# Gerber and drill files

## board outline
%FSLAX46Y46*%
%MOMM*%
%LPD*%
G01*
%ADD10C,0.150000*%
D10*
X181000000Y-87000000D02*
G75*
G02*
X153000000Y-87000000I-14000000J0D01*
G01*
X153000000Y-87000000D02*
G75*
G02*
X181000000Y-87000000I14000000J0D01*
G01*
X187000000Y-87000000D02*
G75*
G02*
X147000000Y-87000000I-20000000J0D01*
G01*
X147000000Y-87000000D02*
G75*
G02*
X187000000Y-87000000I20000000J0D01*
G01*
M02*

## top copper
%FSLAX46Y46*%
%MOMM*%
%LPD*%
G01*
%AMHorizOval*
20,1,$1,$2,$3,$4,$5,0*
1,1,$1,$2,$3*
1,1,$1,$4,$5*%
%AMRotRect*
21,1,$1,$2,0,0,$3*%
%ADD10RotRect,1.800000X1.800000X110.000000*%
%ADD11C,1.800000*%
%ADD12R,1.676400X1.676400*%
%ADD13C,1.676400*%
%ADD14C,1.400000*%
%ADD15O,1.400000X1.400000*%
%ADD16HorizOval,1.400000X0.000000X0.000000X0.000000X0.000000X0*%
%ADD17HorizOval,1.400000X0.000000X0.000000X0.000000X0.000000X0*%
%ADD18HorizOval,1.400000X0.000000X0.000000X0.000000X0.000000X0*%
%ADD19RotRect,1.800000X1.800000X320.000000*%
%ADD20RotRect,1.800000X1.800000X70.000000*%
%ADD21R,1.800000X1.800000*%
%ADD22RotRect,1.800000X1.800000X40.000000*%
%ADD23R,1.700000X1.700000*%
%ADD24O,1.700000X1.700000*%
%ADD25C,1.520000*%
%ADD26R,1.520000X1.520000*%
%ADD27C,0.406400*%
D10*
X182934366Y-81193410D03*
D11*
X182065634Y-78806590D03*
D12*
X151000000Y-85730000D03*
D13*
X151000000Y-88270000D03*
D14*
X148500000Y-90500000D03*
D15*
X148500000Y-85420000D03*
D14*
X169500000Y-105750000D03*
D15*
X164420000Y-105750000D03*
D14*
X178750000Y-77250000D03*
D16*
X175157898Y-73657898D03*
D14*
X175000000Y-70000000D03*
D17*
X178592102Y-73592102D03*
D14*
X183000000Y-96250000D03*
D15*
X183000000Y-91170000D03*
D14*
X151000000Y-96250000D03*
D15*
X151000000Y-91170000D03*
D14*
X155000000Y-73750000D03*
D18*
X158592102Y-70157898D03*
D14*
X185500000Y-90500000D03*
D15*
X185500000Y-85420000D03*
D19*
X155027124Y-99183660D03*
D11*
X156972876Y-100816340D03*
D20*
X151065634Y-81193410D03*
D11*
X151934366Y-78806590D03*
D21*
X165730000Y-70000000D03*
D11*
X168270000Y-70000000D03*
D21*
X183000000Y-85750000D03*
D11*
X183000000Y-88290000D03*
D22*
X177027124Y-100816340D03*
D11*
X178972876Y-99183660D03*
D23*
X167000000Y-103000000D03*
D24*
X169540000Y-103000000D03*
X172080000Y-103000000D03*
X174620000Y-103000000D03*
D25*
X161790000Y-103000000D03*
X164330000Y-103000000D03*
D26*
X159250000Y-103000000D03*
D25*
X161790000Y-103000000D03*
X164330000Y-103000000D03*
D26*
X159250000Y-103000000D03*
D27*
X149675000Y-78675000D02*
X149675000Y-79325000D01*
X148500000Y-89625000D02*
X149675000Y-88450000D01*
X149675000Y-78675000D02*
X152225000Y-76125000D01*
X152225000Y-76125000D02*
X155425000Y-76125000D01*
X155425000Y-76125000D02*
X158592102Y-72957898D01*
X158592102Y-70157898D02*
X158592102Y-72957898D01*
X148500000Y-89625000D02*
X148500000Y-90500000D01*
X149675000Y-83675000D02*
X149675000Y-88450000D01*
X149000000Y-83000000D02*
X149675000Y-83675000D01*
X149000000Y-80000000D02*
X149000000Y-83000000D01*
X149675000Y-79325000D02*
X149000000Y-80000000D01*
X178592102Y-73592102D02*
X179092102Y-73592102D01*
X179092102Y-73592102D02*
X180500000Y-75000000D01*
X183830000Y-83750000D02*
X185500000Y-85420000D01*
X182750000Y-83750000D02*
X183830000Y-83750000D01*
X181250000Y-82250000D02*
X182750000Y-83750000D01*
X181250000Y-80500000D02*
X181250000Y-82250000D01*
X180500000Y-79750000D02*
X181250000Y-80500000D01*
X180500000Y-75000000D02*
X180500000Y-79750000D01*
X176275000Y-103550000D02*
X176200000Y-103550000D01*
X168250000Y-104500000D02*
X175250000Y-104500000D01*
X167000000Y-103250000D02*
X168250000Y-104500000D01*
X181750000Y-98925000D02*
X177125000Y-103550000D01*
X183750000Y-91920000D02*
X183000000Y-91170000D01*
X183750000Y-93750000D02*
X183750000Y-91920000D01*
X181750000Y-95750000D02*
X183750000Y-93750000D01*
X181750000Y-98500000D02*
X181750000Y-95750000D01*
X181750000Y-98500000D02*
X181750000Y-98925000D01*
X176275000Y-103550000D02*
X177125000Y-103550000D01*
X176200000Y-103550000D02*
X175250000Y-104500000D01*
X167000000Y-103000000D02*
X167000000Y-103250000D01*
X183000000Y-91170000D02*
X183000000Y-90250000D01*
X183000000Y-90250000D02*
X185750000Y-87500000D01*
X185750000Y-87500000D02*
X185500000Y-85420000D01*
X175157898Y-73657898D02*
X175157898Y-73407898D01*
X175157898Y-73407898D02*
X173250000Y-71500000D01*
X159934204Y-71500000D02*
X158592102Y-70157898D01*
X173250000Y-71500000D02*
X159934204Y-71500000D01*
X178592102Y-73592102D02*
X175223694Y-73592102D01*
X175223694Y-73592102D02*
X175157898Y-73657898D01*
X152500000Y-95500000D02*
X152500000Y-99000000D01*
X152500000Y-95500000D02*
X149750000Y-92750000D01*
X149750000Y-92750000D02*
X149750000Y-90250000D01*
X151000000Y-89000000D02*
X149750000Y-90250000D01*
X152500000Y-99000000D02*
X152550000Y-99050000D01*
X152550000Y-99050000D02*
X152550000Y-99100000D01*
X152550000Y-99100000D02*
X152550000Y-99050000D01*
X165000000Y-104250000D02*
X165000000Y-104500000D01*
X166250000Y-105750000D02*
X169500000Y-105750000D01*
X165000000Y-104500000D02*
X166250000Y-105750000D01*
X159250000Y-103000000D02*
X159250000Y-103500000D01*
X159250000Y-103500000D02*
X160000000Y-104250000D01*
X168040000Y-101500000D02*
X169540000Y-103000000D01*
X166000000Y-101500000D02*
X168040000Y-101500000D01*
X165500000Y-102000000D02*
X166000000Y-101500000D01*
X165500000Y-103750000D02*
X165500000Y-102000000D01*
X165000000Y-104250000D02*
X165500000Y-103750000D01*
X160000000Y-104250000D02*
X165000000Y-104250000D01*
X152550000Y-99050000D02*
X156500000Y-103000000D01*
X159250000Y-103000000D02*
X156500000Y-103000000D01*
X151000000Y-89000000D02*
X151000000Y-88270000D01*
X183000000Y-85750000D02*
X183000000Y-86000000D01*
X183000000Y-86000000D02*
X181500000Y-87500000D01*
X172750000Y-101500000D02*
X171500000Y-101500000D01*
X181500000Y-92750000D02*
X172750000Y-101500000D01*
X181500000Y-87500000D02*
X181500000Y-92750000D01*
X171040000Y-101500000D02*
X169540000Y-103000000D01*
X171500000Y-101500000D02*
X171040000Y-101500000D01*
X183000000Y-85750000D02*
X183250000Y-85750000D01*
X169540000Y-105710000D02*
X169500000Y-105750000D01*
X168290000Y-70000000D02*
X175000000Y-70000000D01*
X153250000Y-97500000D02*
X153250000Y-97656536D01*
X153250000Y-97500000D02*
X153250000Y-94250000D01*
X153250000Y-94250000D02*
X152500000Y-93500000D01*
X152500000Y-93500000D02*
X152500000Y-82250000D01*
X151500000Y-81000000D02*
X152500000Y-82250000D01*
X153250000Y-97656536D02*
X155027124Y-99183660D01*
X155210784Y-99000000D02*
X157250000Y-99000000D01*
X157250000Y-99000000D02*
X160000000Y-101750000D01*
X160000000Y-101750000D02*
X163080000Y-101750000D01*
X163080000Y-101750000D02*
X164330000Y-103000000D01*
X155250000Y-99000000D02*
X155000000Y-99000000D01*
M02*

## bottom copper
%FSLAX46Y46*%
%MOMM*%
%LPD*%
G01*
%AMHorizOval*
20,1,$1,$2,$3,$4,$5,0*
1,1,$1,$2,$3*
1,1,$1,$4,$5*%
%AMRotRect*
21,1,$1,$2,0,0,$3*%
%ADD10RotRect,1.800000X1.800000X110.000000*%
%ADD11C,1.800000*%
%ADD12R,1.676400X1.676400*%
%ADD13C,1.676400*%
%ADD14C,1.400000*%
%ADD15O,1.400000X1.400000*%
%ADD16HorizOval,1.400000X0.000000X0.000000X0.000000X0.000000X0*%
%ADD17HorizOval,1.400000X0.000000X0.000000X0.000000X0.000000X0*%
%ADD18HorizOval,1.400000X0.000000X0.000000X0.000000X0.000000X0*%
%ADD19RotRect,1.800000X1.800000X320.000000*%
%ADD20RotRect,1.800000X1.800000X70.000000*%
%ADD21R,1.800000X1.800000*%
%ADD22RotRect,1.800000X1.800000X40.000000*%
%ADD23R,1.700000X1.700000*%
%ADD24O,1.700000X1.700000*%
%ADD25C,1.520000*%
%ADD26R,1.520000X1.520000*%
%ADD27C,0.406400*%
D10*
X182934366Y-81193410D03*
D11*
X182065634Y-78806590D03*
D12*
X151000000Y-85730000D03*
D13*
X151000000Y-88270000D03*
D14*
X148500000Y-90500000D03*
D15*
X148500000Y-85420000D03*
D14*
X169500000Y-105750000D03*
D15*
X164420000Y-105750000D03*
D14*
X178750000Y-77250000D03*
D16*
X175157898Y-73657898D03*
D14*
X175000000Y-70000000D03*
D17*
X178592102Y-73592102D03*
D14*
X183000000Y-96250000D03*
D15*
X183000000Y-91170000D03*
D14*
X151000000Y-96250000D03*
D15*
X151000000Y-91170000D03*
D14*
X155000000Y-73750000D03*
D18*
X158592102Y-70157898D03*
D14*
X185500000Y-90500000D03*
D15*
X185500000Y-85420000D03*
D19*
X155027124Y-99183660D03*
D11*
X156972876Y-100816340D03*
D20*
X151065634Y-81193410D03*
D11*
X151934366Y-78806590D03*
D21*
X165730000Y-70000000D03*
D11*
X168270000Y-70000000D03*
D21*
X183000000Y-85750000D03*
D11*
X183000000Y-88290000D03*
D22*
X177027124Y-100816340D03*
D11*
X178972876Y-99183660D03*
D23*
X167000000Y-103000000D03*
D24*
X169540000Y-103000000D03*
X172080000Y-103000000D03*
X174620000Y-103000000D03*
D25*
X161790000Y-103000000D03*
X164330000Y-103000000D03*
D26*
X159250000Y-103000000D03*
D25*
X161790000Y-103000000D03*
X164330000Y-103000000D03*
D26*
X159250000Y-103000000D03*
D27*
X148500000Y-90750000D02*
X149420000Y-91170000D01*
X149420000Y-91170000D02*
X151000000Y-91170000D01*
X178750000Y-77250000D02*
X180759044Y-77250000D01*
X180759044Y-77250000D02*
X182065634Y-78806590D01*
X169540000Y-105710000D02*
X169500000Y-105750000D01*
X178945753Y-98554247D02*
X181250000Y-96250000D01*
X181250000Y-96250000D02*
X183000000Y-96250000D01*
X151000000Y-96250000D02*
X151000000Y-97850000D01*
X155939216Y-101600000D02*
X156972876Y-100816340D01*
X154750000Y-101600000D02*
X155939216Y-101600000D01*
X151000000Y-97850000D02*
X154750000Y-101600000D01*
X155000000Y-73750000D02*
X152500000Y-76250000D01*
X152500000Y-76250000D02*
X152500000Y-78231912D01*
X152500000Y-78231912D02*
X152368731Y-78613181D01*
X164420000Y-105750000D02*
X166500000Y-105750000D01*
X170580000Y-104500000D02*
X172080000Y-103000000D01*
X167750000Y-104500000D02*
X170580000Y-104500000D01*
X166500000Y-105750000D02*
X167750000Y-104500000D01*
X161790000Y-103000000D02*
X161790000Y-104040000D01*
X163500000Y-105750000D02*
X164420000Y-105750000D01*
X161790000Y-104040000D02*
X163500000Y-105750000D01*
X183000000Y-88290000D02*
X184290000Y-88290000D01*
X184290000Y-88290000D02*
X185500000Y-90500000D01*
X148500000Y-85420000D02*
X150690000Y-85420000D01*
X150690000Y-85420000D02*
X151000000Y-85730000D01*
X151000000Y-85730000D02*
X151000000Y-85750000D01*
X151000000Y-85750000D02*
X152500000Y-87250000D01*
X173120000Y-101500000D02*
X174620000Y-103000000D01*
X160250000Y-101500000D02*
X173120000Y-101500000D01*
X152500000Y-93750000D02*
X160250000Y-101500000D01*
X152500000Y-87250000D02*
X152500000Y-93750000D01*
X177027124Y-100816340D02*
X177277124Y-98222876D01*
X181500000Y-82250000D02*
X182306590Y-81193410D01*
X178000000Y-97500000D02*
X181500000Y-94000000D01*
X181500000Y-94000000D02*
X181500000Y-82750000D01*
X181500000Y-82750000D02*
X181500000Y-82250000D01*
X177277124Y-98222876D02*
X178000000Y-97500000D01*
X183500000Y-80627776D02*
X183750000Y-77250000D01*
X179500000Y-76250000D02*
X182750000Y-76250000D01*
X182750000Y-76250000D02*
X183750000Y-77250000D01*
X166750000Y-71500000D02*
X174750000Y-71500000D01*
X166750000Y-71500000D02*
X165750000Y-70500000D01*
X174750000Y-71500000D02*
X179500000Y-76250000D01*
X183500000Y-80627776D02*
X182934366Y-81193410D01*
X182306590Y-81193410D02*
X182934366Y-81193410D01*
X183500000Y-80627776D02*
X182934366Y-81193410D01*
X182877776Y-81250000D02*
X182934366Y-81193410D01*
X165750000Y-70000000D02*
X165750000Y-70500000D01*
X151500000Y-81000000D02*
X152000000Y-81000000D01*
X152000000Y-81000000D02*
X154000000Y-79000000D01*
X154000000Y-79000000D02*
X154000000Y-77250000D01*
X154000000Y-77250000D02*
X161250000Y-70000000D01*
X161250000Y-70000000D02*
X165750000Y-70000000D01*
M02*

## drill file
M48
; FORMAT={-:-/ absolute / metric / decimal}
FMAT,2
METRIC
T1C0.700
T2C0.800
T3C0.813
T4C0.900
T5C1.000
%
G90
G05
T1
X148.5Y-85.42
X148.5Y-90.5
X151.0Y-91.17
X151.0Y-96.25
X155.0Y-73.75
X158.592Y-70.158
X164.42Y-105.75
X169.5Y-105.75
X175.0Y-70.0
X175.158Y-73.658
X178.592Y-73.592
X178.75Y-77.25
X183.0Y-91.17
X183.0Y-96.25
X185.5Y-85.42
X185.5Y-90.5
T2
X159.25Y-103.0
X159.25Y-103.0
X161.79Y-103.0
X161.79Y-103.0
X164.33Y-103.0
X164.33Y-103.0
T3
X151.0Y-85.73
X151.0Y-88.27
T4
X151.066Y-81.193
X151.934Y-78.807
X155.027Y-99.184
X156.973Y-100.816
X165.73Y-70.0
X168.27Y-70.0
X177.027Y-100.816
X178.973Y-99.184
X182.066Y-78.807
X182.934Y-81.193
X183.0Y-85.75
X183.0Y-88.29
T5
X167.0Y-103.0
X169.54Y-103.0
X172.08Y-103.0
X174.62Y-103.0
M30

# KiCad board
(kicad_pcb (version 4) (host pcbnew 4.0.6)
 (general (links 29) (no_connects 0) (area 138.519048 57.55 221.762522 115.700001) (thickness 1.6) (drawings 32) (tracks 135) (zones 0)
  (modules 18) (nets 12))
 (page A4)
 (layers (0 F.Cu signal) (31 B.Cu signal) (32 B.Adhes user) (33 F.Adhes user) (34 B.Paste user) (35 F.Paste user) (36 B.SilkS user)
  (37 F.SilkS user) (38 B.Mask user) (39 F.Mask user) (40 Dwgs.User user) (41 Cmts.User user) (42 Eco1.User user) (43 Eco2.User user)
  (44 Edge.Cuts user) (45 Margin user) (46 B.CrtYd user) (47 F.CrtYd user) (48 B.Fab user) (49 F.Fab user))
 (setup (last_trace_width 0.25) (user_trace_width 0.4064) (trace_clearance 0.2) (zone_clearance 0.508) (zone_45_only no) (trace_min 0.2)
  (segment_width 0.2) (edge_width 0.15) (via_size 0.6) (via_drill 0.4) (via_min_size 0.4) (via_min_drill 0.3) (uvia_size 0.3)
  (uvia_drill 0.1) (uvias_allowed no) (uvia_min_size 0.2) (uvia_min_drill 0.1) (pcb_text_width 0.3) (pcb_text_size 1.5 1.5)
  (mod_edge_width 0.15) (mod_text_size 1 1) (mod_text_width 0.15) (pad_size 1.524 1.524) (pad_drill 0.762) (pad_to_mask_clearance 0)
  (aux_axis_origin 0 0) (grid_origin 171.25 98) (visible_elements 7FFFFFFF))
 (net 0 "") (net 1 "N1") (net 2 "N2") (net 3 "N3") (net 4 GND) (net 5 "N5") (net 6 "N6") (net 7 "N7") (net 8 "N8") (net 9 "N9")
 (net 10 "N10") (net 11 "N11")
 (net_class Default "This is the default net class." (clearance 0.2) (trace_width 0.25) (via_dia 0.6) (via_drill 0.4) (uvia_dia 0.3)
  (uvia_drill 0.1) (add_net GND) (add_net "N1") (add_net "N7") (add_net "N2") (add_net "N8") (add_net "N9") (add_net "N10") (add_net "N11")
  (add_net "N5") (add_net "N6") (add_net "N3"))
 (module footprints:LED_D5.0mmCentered (layer F.Cu) (at 182.5 80 110)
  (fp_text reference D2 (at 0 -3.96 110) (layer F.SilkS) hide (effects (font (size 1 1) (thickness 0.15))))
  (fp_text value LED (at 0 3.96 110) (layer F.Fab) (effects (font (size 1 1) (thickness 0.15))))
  (pad 1 thru_hole rect (at -1.27 0 110) (size 1.8 1.8) (drill 0.9) (layers *.Cu *.Mask) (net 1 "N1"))
  (pad 2 thru_hole circle (at 1.27 0 110) (size 1.8 1.8) (drill 0.9) (layers *.Cu *.Mask) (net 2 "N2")))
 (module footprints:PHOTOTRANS (layer F.Cu) (at 151 87 270)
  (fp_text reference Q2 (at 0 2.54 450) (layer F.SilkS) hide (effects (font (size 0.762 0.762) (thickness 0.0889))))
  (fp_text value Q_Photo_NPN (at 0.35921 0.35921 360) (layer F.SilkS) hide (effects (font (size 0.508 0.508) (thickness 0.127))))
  (pad 1 thru_hole rect (at -1.27 0 270) (size 1.6764 1.6764) (drill 0.8128) (layers *.Cu *.Mask F.SilkS) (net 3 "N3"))
  (pad 2 thru_hole circle (at 1.27 0 315) (size 1.6764 1.6764) (drill 0.8128) (layers *.Cu *.Mask F.SilkS) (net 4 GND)))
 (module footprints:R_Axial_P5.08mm (layer F.Cu) (at 148.5 90.5 90)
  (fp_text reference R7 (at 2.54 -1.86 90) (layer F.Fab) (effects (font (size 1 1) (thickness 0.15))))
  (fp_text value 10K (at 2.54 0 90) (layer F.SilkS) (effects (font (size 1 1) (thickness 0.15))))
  (pad 1 thru_hole circle (at 0 0 90) (size 1.4 1.4) (drill 0.7) (layers *.Cu *.Mask) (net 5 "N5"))
  (pad 2 thru_hole oval (at 5.08 0 90) (size 1.4 1.4) (drill 0.7) (layers *.Cu *.Mask) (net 3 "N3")))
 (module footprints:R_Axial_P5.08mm (layer F.Cu) (at 169.5 105.75 180)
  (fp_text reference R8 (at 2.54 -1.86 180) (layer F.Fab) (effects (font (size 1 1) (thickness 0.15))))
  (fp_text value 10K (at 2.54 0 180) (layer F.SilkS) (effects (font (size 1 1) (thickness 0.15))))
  (pad 1 thru_hole circle (at 0 0 180) (size 1.4 1.4) (drill 0.7) (layers *.Cu *.Mask) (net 4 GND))
  (pad 2 thru_hole oval (at 5.08 0 180) (size 1.4 1.4) (drill 0.7) (layers *.Cu *.Mask) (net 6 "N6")))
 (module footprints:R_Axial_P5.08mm (layer F.Cu) (at 178.75 77.25 135)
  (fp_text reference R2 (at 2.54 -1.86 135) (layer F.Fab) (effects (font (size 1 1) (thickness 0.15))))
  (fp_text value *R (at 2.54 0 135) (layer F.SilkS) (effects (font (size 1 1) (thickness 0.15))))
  (pad 1 thru_hole circle (at 0 0 135) (size 1.4 1.4) (drill 0.7) (layers *.Cu *.Mask) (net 2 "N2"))
  (pad 2 thru_hole oval (at 5.08 0 135) (size 1.4 1.4) (drill 0.7) (layers *.Cu *.Mask) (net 5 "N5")))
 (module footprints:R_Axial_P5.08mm (layer F.Cu) (at 175 70 315)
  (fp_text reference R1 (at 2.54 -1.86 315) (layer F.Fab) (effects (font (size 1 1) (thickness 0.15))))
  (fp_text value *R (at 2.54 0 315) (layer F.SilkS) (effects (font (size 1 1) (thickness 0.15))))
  (pad 1 thru_hole circle (at 0 0 315) (size 1.4 1.4) (drill 0.7) (layers *.Cu *.Mask) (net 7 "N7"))
  (pad 2 thru_hole oval (at 5.08 0 315) (size 1.4 1.4) (drill 0.7) (layers *.Cu *.Mask) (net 5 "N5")))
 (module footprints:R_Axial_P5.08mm (layer F.Cu) (at 183 96.25 90)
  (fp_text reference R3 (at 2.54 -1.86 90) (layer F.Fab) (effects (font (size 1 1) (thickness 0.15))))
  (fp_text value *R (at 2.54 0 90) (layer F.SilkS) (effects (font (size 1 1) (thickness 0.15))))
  (pad 1 thru_hole circle (at 0 0 90) (size 1.4 1.4) (drill 0.7) (layers *.Cu *.Mask) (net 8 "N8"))
  (pad 2 thru_hole oval (at 5.08 0 90) (size 1.4 1.4) (drill 0.7) (layers *.Cu *.Mask) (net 5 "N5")))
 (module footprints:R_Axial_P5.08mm (layer F.Cu) (at 151 96.25 90)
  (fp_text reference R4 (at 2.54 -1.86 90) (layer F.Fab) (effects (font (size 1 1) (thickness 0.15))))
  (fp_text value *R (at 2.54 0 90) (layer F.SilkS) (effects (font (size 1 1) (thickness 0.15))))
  (pad 1 thru_hole circle (at 0 0 90) (size 1.4 1.4) (drill 0.7) (layers *.Cu *.Mask) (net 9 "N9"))
  (pad 2 thru_hole oval (at 5.08 0 90) (size 1.4 1.4) (drill 0.7) (layers *.Cu *.Mask) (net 5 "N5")))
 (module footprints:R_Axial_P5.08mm (layer F.Cu) (at 155 73.75 45)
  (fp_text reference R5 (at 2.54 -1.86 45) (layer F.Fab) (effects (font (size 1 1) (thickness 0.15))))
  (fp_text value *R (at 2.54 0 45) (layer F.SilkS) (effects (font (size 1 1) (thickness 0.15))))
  (pad 1 thru_hole circle (at 0 0 45) (size 1.4 1.4) (drill 0.7) (layers *.Cu *.Mask) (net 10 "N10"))
  (pad 2 thru_hole oval (at 5.08 0 45) (size 1.4 1.4) (drill 0.7) (layers *.Cu *.Mask) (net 5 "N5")))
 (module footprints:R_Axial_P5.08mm (layer F.Cu) (at 185.5 90.5 90)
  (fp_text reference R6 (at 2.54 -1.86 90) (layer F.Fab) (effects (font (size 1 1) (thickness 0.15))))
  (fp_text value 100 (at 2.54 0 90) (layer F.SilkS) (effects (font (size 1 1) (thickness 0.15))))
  (pad 1 thru_hole circle (at 0 0 90) (size 1.4 1.4) (drill 0.7) (layers *.Cu *.Mask) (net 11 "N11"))
  (pad 2 thru_hole oval (at 5.08 0 90) (size 1.4 1.4) (drill 0.7) (layers *.Cu *.Mask) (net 5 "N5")))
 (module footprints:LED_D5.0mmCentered (layer F.Cu) (at 156 100 320)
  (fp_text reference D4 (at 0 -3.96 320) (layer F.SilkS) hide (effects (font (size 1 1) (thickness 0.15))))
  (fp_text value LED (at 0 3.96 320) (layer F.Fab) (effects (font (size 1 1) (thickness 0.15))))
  (pad 1 thru_hole rect (at -1.27 0 320) (size 1.8 1.8) (drill 0.9) (layers *.Cu *.Mask) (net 1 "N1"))
  (pad 2 thru_hole circle (at 1.27 0 320) (size 1.8 1.8) (drill 0.9) (layers *.Cu *.Mask) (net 9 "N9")))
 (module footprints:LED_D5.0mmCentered (layer F.Cu) (at 151.5 80 70)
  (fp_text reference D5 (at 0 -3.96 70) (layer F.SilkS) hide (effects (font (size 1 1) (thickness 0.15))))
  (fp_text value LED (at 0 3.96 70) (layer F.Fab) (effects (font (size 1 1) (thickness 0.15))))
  (pad 1 thru_hole rect (at -1.27 0 70) (size 1.8 1.8) (drill 0.9) (layers *.Cu *.Mask) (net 1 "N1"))
  (pad 2 thru_hole circle (at 1.27 0 70) (size 1.8 1.8) (drill 0.9) (layers *.Cu *.Mask) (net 10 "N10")))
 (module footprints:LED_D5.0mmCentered (layer F.Cu) (at 167 70)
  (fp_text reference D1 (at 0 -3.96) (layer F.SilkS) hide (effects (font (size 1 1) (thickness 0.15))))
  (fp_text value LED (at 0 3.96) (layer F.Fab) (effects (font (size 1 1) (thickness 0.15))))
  (pad 1 thru_hole rect (at -1.27 0) (size 1.8 1.8) (drill 0.9) (layers *.Cu *.Mask) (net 1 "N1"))
  (pad 2 thru_hole circle (at 1.27 0) (size 1.8 1.8) (drill 0.9) (layers *.Cu *.Mask) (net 7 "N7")))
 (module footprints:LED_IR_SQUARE (layer F.Cu) (at 183 85.75 270)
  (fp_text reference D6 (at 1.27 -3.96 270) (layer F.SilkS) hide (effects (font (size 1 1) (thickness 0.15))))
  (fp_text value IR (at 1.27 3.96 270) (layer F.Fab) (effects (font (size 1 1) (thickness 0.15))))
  (pad 1 thru_hole rect (at 0 0 270) (size 1.8 1.8) (drill 0.9) (layers *.Cu *.Mask) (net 4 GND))
  (pad 2 thru_hole circle (at 2.54 0 270) (size 1.8 1.8) (drill 0.9) (layers *.Cu *.Mask) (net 11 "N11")))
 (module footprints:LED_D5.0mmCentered (layer F.Cu) (at 178 100 40)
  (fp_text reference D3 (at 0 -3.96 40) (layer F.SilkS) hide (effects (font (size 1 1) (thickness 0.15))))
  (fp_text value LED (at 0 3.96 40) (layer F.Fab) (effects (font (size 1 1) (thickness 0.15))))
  (pad 1 thru_hole rect (at -1.27 0 40) (size 1.8 1.8) (drill 0.9) (layers *.Cu *.Mask) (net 1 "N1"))
  (pad 2 thru_hole circle (at 1.27 0 40) (size 1.8 1.8) (drill 0.9) (layers *.Cu *.Mask) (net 8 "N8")))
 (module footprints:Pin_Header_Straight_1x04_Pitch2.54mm (layer F.Cu) (at 167 103 90)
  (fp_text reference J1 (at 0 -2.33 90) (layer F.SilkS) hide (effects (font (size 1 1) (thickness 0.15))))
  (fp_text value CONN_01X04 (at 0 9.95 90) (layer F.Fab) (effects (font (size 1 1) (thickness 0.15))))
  (pad 1 thru_hole rect (at 0 0 90) (size 1.7 1.7) (drill 1) (layers *.Cu *.Mask) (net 5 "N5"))
  (pad 2 thru_hole oval (at 0 2.54 90) (size 1.7 1.7) (drill 1) (layers *.Cu *.Mask) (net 4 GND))
  (pad 3 thru_hole oval (at 0 5.08 90) (size 1.7 1.7) (drill 1) (layers *.Cu *.Mask) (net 6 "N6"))
  (pad 4 thru_hole oval (at 0 7.62 90) (size 1.7 1.7) (drill 1) (layers *.Cu *.Mask) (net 3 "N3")))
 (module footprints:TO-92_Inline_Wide (layer B.Cu) (at 159.25 103)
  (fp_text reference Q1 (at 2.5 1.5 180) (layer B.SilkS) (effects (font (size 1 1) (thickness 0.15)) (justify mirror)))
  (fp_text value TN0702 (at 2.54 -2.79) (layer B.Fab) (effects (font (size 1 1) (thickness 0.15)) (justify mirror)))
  (pad 2 thru_hole circle (at 2.54 0 270) (size 1.52 1.52) (drill 0.8) (layers *.Cu *.Mask) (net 6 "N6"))
  (pad 3 thru_hole circle (at 5.08 0 270) (size 1.52 1.52) (drill 0.8) (layers *.Cu *.Mask) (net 1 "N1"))
  (pad 1 thru_hole rect (at 0 0 270) (size 1.52 1.52) (drill 0.8) (layers *.Cu *.Mask) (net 4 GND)))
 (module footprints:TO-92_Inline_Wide (layer F.Cu) (at 159.25 103)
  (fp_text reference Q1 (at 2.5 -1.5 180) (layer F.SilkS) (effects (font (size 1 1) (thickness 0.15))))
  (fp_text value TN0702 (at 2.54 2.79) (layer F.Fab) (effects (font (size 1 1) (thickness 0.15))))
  (pad 2 thru_hole circle (at 2.54 0 90) (size 1.52 1.52) (drill 0.8) (layers *.Cu *.Mask) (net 6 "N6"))
  (pad 3 thru_hole circle (at 5.08 0 90) (size 1.52 1.52) (drill 0.8) (layers *.Cu *.Mask) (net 1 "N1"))
  (pad 1 thru_hole rect (at 0 0 90) (size 1.52 1.52) (drill 0.8) (layers *.Cu *.Mask) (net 4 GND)))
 (gr_circle (center 167 87) (end 181 87) (layer Edge.Cuts) (width 0.15))
 (gr_circle (center 167 87) (end 187 87) (layer Edge.Cuts) (width 0.15))
 (segment (start 149.675 78.675) (end 149.675 79.325) (width 0.4064) (layer F.Cu) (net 5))
 (segment (start 148.5 89.625) (end 149.675 88.45) (width 0.4064) (layer F.Cu) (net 5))
 (segment (start 149.675 78.675) (end 152.225 76.125) (width 0.4064) (layer F.Cu) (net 5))
 (segment (start 152.225 76.125) (end 155.425 76.125) (width 0.4064) (layer F.Cu) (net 5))
 (segment (start 155.425 76.125) (end 158.592102 72.957898) (width 0.4064) (layer F.Cu) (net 5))
 (segment (start 158.592102 70.157898) (end 158.592102 72.957898) (width 0.4064) (layer F.Cu) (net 5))
 (segment (start 148.5 89.625) (end 148.5 90.5) (width 0.4064) (layer F.Cu) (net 5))
 (segment (start 149.675 83.675) (end 149.675 88.45) (width 0.4064) (layer F.Cu) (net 5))
 (segment (start 149 83) (end 149.675 83.675) (width 0.4064) (layer F.Cu) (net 5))
 (segment (start 149 80) (end 149 83) (width 0.4064) (layer F.Cu) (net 5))
 (segment (start 149.675 79.325) (end 149 80) (width 0.4064) (layer F.Cu) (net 5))
 (segment (start 178.592102 73.592102) (end 179.092102 73.592102) (width 0.4064) (layer F.Cu) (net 5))
 (segment (start 179.092102 73.592102) (end 180.5 75) (width 0.4064) (layer F.Cu) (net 5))
 (segment (start 183.83 83.75) (end 185.5 85.42) (width 0.4064) (layer F.Cu) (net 5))
 (segment (start 182.75 83.75) (end 183.83 83.75) (width 0.4064) (layer F.Cu) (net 5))
 (segment (start 181.25 82.25) (end 182.75 83.75) (width 0.4064) (layer F.Cu) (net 5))
 (segment (start 181.25 80.5) (end 181.25 82.25) (width 0.4064) (layer F.Cu) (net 5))
 (segment (start 180.5 79.75) (end 181.25 80.5) (width 0.4064) (layer F.Cu) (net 5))
 (segment (start 180.5 75) (end 180.5 79.75) (width 0.4064) (layer F.Cu) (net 5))
 (segment (start 176.275 103.55) (end 176.2 103.55) (width 0.4064) (layer F.Cu) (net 5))
 (segment (start 168.25 104.5) (end 175.25 104.5) (width 0.4064) (layer F.Cu) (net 5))
 (segment (start 167 103.25) (end 168.25 104.5) (width 0.4064) (layer F.Cu) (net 5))
 (segment (start 181.75 98.925) (end 177.125 103.55) (width 0.4064) (layer F.Cu) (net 5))
 (segment (start 183.75 91.92) (end 183 91.17) (width 0.4064) (layer F.Cu) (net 5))
 (segment (start 183.75 93.75) (end 183.75 91.92) (width 0.4064) (layer F.Cu) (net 5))
 (segment (start 181.75 95.75) (end 183.75 93.75) (width 0.4064) (layer F.Cu) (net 5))
 (segment (start 181.75 98.5) (end 181.75 95.75) (width 0.4064) (layer F.Cu) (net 5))
 (segment (start 181.75 98.5) (end 181.75 98.925) (width 0.4064) (layer F.Cu) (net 5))
 (segment (start 176.275 103.55) (end 177.125 103.55) (width 0.4064) (layer F.Cu) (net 5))
 (segment (start 176.2 103.55) (end 175.25 104.5) (width 0.4064) (layer F.Cu) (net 5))
 (segment (start 148.5 90.75) (end 149.42 91.17) (width 0.4064) (layer B.Cu) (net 5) (status 10))
 (segment (start 149.42 91.17) (end 151 91.17) (width 0.4064) (layer B.Cu) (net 5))
 (segment (start 167 103) (end 167 103.25) (width 0.4064) (layer F.Cu) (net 5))
 (segment (start 183 91.17) (end 183 90.25) (width 0.4064) (layer F.Cu) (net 5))
 (segment (start 183 90.25) (end 185.75 87.5) (width 0.4064) (layer F.Cu) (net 5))
 (segment (start 185.75 87.5) (end 185.5 85.42) (width 0.4064) (layer F.Cu) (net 5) (status 20))
 (segment (start 175.157898 73.657898) (end 175.157898 73.407898) (width 0.4064) (layer F.Cu) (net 5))
 (segment (start 175.157898 73.407898) (end 173.25 71.5) (width 0.4064) (layer F.Cu) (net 5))
 (segment (start 159.934204 71.5) (end 158.592102 70.157898) (width 0.4064) (layer F.Cu) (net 5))
 (segment (start 173.25 71.5) (end 159.934204 71.5) (width 0.4064) (layer F.Cu) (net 5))
 (segment (start 178.592102 73.592102) (end 175.223694 73.592102) (width 0.4064) (layer F.Cu) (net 5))
 (segment (start 175.223694 73.592102) (end 175.157898 73.657898) (width 0.4064) (layer F.Cu) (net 5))
 (segment (start 178.75 77.25) (end 180.759044 77.25) (width 0.4064) (layer B.Cu) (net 2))
 (segment (start 180.759044 77.25) (end 182.065634 78.80659) (width 0.4064) (layer B.Cu) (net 2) (status 20))
 (segment (start 152.5 95.5) (end 152.5 99) (width 0.4064) (layer F.Cu) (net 4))
 (segment (start 152.5 95.5) (end 149.75 92.75) (width 0.4064) (layer F.Cu) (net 4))
 (segment (start 149.75 92.75) (end 149.75 90.25) (width 0.4064) (layer F.Cu) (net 4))
 (segment (start 151 89) (end 149.75 90.25) (width 0.4064) (layer F.Cu) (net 4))
 (segment (start 152.5 99) (end 152.55 99.05) (width 0.4064) (layer F.Cu) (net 4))
 (segment (start 152.55 99.05) (end 152.55 99.1) (width 0.4064) (layer F.Cu) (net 4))
 (segment (start 152.55 99.1) (end 152.55 99.05) (width 0.4064) (layer F.Cu) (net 4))
 (segment (start 165 104.25) (end 165 104.5) (width 0.4064) (layer F.Cu) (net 4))
 (segment (start 166.25 105.75) (end 169.5 105.75) (width 0.4064) (layer F.Cu) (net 4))
 (segment (start 165 104.5) (end 166.25 105.75) (width 0.4064) (layer F.Cu) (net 4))
 (segment (start 159.25 103) (end 159.25 103.5) (width 0.4064) (layer F.Cu) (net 4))
 (segment (start 159.25 103.5) (end 160 104.25) (width 0.4064) (layer F.Cu) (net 4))
 (segment (start 168.04 101.5) (end 169.54 103) (width 0.4064) (layer F.Cu) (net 4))
 (segment (start 166 101.5) (end 168.04 101.5) (width 0.4064) (layer F.Cu) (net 4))
 (segment (start 165.5 102) (end 166 101.5) (width 0.4064) (layer F.Cu) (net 4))
 (segment (start 165.5 103.75) (end 165.5 102) (width 0.4064) (layer F.Cu) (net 4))
 (segment (start 165 104.25) (end 165.5 103.75) (width 0.4064) (layer F.Cu) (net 4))
 (segment (start 160 104.25) (end 165 104.25) (width 0.4064) (layer F.Cu) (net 4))
 (segment (start 152.55 99.05) (end 156.5 103) (width 0.4064) (layer F.Cu) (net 4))
 (segment (start 159.25 103) (end 156.5 103) (width 0.4064) (layer F.Cu) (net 4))
 (segment (start 151 89) (end 151 88.27) (width 0.4064) (layer F.Cu) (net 4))
 (segment (start 169.54 105.71) (end 169.5 105.75) (width 0.4064) (layer B.Cu) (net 4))
 (segment (start 183 85.75) (end 183 86) (width 0.4064) (layer F.Cu) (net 4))
 (segment (start 183 86) (end 181.5 87.5) (width 0.4064) (layer F.Cu) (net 4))
 (segment (start 172.75 101.5) (end 171.5 101.5) (width 0.4064) (layer F.Cu) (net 4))
 (segment (start 181.5 92.75) (end 172.75 101.5) (width 0.4064) (layer F.Cu) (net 4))
 (segment (start 181.5 87.5) (end 181.5 92.75) (width 0.4064) (layer F.Cu) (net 4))
 (segment (start 171.04 101.5) (end 169.54 103) (width 0.4064) (layer F.Cu) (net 4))
 (segment (start 171.5 101.5) (end 171.04 101.5) (width 0.4064) (layer F.Cu) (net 4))
 (segment (start 183 85.75) (end 183.25 85.75) (width 0.4064) (layer F.Cu) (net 4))
 (segment (start 169.54 105.71) (end 169.5 105.75) (width 0.4064) (layer F.Cu) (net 4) (status 30))
 (segment (start 168.29 70) (end 175 70) (width 0.4064) (layer F.Cu) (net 7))
 (segment (start 178.945753 98.554247) (end 181.25 96.25) (width 0.4064) (layer B.Cu) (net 8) (status 10))
 (segment (start 181.25 96.25) (end 183 96.25) (width 0.4064) (layer B.Cu) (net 8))
 (segment (start 151 96.25) (end 151 97.85) (width 0.4064) (layer B.Cu) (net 9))
 (segment (start 155.939216 101.6) (end 156.972876 100.81634) (width 0.4064) (layer B.Cu) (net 9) (status 20))
 (segment (start 154.75 101.6) (end 155.939216 101.6) (width 0.4064) (layer B.Cu) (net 9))
 (segment (start 151 97.85) (end 154.75 101.6) (width 0.4064) (layer B.Cu) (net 9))
 (segment (start 155 73.75) (end 152.5 76.25) (width 0.4064) (layer B.Cu) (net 10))
 (segment (start 152.5 76.25) (end 152.5 78.231912) (width 0.4064) (layer B.Cu) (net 10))
 (segment (start 152.5 78.231912) (end 152.368731 78.613181) (width 0.4064) (layer B.Cu) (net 10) (status 20))
 (segment (start 164.42 105.75) (end 166.5 105.75) (width 0.4064) (layer B.Cu) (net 6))
 (segment (start 170.58 104.5) (end 172.08 103) (width 0.4064) (layer B.Cu) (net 6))
 (segment (start 167.75 104.5) (end 170.58 104.5) (width 0.4064) (layer B.Cu) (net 6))
 (segment (start 166.5 105.75) (end 167.75 104.5) (width 0.4064) (layer B.Cu) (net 6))
 (segment (start 161.79 103) (end 161.79 104.04) (width 0.4064) (layer B.Cu) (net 6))
 (segment (start 163.5 105.75) (end 164.42 105.75) (width 0.4064) (layer B.Cu) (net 6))
 (segment (start 161.79 104.04) (end 163.5 105.75) (width 0.4064) (layer B.Cu) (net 6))
 (segment (start 183 88.29) (end 184.29 88.29) (width 0.4064) (layer B.Cu) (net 11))
 (segment (start 184.29 88.29) (end 185.5 90.5) (width 0.4064) (layer B.Cu) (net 11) (status 20))
 (segment (start 148.5 85.42) (end 150.69 85.42) (width 0.4064) (layer B.Cu) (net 3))
 (segment (start 150.69 85.42) (end 151 85.73) (width 0.4064) (layer B.Cu) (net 3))
 (segment (start 151 85.73) (end 151 85.75) (width 0.4064) (layer B.Cu) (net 3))
 (segment (start 151 85.75) (end 152.5 87.25) (width 0.4064) (layer B.Cu) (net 3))
 (segment (start 173.12 101.5) (end 174.62 103) (width 0.4064) (layer B.Cu) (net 3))
 (segment (start 160.25 101.5) (end 173.12 101.5) (width 0.4064) (layer B.Cu) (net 3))
 (segment (start 152.5 93.75) (end 160.25 101.5) (width 0.4064) (layer B.Cu) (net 3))
 (segment (start 152.5 87.25) (end 152.5 93.75) (width 0.4064) (layer B.Cu) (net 3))
 (segment (start 177.027124 100.81634) (end 177.277124 98.222876) (width 0.4064) (layer B.Cu) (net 1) (status 10))
 (segment (start 181.5 82.25) (end 182.30659 81.19341) (width 0.4064) (layer B.Cu) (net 1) (status 20))
 (segment (start 178 97.5) (end 181.5 94) (width 0.4064) (layer B.Cu) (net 1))
 (segment (start 181.5 94) (end 181.5 82.75) (width 0.4064) (layer B.Cu) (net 1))
 (segment (start 181.5 82.75) (end 181.5 82.25) (width 0.4064) (layer B.Cu) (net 1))
 (segment (start 177.277124 98.222876) (end 178 97.5) (width 0.4064) (layer B.Cu) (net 1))
 (segment (start 183.5 80.627776) (end 183.75 77.25) (width 0.4064) (layer B.Cu) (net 1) (status 10))
 (segment (start 179.5 76.25) (end 182.75 76.25) (width 0.4064) (layer B.Cu) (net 1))
 (segment (start 182.75 76.25) (end 183.75 77.25) (width 0.4064) (layer B.Cu) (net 1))
 (segment (start 166.75 71.5) (end 174.75 71.5) (width 0.4064) (layer B.Cu) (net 1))
 (segment (start 166.75 71.5) (end 165.75 70.5) (width 0.4064) (layer B.Cu) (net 1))
 (segment (start 174.75 71.5) (end 179.5 76.25) (width 0.4064) (layer B.Cu) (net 1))
 (segment (start 183.5 80.627776) (end 182.934366 81.19341) (width 0.4064) (layer B.Cu) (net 1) (status 30))
 (segment (start 182.30659 81.19341) (end 182.934366 81.19341) (width 0.4064) (layer B.Cu) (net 1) (status 30))
 (segment (start 183.5 80.627776) (end 182.934366 81.19341) (width 0.4064) (layer B.Cu) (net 1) (status 30))
 (segment (start 182.877776 81.25) (end 182.934366 81.19341) (width 0.4064) (layer B.Cu) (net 1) (status 30))
 (segment (start 153.25 97.5) (end 153.25 97.656536) (width 0.4064) (layer F.Cu) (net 1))
 (segment (start 153.25 97.5) (end 153.25 94.25) (width 0.4064) (layer F.Cu) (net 1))
 (segment (start 153.25 94.25) (end 152.5 93.5) (width 0.4064) (layer F.Cu) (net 1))
 (segment (start 152.5 93.5) (end 152.5 82.25) (width 0.4064) (layer F.Cu) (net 1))
 (segment (start 151.5 81) (end 152.5 82.25) (width 0.4064) (layer F.Cu) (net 1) (status 10))
 (segment (start 153.25 97.656536) (end 155.027124 99.18366) (width 0.4064) (layer F.Cu) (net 1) (status 20))
 (segment (start 155.210784 99) (end 157.25 99) (width 0.4064) (layer F.Cu) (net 1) (status 10))
 (segment (start 157.25 99) (end 160 101.75) (width 0.4064) (layer F.Cu) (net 1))
 (segment (start 160 101.75) (end 163.08 101.75) (width 0.4064) (layer F.Cu) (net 1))
 (segment (start 163.08 101.75) (end 164.33 103) (width 0.4064) (layer F.Cu) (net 1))
 (segment (start 155.25 99) (end 155 99) (width 0.4064) (layer F.Cu) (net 1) (status 30))
 (segment (start 165.75 70) (end 165.75 70.5) (width 0.4064) (layer B.Cu) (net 1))
 (segment (start 151.5 81) (end 152 81) (width 0.4064) (layer B.Cu) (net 1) (status 10))
 (segment (start 152 81) (end 154 79) (width 0.4064) (layer B.Cu) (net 1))
 (segment (start 154 79) (end 154 77.25) (width 0.4064) (layer B.Cu) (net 1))
 (segment (start 154 77.25) (end 161.25 70) (width 0.4064) (layer B.Cu) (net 1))
 (segment (start 161.25 70) (end 165.75 70) (width 0.4064) (layer B.Cu) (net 1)))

